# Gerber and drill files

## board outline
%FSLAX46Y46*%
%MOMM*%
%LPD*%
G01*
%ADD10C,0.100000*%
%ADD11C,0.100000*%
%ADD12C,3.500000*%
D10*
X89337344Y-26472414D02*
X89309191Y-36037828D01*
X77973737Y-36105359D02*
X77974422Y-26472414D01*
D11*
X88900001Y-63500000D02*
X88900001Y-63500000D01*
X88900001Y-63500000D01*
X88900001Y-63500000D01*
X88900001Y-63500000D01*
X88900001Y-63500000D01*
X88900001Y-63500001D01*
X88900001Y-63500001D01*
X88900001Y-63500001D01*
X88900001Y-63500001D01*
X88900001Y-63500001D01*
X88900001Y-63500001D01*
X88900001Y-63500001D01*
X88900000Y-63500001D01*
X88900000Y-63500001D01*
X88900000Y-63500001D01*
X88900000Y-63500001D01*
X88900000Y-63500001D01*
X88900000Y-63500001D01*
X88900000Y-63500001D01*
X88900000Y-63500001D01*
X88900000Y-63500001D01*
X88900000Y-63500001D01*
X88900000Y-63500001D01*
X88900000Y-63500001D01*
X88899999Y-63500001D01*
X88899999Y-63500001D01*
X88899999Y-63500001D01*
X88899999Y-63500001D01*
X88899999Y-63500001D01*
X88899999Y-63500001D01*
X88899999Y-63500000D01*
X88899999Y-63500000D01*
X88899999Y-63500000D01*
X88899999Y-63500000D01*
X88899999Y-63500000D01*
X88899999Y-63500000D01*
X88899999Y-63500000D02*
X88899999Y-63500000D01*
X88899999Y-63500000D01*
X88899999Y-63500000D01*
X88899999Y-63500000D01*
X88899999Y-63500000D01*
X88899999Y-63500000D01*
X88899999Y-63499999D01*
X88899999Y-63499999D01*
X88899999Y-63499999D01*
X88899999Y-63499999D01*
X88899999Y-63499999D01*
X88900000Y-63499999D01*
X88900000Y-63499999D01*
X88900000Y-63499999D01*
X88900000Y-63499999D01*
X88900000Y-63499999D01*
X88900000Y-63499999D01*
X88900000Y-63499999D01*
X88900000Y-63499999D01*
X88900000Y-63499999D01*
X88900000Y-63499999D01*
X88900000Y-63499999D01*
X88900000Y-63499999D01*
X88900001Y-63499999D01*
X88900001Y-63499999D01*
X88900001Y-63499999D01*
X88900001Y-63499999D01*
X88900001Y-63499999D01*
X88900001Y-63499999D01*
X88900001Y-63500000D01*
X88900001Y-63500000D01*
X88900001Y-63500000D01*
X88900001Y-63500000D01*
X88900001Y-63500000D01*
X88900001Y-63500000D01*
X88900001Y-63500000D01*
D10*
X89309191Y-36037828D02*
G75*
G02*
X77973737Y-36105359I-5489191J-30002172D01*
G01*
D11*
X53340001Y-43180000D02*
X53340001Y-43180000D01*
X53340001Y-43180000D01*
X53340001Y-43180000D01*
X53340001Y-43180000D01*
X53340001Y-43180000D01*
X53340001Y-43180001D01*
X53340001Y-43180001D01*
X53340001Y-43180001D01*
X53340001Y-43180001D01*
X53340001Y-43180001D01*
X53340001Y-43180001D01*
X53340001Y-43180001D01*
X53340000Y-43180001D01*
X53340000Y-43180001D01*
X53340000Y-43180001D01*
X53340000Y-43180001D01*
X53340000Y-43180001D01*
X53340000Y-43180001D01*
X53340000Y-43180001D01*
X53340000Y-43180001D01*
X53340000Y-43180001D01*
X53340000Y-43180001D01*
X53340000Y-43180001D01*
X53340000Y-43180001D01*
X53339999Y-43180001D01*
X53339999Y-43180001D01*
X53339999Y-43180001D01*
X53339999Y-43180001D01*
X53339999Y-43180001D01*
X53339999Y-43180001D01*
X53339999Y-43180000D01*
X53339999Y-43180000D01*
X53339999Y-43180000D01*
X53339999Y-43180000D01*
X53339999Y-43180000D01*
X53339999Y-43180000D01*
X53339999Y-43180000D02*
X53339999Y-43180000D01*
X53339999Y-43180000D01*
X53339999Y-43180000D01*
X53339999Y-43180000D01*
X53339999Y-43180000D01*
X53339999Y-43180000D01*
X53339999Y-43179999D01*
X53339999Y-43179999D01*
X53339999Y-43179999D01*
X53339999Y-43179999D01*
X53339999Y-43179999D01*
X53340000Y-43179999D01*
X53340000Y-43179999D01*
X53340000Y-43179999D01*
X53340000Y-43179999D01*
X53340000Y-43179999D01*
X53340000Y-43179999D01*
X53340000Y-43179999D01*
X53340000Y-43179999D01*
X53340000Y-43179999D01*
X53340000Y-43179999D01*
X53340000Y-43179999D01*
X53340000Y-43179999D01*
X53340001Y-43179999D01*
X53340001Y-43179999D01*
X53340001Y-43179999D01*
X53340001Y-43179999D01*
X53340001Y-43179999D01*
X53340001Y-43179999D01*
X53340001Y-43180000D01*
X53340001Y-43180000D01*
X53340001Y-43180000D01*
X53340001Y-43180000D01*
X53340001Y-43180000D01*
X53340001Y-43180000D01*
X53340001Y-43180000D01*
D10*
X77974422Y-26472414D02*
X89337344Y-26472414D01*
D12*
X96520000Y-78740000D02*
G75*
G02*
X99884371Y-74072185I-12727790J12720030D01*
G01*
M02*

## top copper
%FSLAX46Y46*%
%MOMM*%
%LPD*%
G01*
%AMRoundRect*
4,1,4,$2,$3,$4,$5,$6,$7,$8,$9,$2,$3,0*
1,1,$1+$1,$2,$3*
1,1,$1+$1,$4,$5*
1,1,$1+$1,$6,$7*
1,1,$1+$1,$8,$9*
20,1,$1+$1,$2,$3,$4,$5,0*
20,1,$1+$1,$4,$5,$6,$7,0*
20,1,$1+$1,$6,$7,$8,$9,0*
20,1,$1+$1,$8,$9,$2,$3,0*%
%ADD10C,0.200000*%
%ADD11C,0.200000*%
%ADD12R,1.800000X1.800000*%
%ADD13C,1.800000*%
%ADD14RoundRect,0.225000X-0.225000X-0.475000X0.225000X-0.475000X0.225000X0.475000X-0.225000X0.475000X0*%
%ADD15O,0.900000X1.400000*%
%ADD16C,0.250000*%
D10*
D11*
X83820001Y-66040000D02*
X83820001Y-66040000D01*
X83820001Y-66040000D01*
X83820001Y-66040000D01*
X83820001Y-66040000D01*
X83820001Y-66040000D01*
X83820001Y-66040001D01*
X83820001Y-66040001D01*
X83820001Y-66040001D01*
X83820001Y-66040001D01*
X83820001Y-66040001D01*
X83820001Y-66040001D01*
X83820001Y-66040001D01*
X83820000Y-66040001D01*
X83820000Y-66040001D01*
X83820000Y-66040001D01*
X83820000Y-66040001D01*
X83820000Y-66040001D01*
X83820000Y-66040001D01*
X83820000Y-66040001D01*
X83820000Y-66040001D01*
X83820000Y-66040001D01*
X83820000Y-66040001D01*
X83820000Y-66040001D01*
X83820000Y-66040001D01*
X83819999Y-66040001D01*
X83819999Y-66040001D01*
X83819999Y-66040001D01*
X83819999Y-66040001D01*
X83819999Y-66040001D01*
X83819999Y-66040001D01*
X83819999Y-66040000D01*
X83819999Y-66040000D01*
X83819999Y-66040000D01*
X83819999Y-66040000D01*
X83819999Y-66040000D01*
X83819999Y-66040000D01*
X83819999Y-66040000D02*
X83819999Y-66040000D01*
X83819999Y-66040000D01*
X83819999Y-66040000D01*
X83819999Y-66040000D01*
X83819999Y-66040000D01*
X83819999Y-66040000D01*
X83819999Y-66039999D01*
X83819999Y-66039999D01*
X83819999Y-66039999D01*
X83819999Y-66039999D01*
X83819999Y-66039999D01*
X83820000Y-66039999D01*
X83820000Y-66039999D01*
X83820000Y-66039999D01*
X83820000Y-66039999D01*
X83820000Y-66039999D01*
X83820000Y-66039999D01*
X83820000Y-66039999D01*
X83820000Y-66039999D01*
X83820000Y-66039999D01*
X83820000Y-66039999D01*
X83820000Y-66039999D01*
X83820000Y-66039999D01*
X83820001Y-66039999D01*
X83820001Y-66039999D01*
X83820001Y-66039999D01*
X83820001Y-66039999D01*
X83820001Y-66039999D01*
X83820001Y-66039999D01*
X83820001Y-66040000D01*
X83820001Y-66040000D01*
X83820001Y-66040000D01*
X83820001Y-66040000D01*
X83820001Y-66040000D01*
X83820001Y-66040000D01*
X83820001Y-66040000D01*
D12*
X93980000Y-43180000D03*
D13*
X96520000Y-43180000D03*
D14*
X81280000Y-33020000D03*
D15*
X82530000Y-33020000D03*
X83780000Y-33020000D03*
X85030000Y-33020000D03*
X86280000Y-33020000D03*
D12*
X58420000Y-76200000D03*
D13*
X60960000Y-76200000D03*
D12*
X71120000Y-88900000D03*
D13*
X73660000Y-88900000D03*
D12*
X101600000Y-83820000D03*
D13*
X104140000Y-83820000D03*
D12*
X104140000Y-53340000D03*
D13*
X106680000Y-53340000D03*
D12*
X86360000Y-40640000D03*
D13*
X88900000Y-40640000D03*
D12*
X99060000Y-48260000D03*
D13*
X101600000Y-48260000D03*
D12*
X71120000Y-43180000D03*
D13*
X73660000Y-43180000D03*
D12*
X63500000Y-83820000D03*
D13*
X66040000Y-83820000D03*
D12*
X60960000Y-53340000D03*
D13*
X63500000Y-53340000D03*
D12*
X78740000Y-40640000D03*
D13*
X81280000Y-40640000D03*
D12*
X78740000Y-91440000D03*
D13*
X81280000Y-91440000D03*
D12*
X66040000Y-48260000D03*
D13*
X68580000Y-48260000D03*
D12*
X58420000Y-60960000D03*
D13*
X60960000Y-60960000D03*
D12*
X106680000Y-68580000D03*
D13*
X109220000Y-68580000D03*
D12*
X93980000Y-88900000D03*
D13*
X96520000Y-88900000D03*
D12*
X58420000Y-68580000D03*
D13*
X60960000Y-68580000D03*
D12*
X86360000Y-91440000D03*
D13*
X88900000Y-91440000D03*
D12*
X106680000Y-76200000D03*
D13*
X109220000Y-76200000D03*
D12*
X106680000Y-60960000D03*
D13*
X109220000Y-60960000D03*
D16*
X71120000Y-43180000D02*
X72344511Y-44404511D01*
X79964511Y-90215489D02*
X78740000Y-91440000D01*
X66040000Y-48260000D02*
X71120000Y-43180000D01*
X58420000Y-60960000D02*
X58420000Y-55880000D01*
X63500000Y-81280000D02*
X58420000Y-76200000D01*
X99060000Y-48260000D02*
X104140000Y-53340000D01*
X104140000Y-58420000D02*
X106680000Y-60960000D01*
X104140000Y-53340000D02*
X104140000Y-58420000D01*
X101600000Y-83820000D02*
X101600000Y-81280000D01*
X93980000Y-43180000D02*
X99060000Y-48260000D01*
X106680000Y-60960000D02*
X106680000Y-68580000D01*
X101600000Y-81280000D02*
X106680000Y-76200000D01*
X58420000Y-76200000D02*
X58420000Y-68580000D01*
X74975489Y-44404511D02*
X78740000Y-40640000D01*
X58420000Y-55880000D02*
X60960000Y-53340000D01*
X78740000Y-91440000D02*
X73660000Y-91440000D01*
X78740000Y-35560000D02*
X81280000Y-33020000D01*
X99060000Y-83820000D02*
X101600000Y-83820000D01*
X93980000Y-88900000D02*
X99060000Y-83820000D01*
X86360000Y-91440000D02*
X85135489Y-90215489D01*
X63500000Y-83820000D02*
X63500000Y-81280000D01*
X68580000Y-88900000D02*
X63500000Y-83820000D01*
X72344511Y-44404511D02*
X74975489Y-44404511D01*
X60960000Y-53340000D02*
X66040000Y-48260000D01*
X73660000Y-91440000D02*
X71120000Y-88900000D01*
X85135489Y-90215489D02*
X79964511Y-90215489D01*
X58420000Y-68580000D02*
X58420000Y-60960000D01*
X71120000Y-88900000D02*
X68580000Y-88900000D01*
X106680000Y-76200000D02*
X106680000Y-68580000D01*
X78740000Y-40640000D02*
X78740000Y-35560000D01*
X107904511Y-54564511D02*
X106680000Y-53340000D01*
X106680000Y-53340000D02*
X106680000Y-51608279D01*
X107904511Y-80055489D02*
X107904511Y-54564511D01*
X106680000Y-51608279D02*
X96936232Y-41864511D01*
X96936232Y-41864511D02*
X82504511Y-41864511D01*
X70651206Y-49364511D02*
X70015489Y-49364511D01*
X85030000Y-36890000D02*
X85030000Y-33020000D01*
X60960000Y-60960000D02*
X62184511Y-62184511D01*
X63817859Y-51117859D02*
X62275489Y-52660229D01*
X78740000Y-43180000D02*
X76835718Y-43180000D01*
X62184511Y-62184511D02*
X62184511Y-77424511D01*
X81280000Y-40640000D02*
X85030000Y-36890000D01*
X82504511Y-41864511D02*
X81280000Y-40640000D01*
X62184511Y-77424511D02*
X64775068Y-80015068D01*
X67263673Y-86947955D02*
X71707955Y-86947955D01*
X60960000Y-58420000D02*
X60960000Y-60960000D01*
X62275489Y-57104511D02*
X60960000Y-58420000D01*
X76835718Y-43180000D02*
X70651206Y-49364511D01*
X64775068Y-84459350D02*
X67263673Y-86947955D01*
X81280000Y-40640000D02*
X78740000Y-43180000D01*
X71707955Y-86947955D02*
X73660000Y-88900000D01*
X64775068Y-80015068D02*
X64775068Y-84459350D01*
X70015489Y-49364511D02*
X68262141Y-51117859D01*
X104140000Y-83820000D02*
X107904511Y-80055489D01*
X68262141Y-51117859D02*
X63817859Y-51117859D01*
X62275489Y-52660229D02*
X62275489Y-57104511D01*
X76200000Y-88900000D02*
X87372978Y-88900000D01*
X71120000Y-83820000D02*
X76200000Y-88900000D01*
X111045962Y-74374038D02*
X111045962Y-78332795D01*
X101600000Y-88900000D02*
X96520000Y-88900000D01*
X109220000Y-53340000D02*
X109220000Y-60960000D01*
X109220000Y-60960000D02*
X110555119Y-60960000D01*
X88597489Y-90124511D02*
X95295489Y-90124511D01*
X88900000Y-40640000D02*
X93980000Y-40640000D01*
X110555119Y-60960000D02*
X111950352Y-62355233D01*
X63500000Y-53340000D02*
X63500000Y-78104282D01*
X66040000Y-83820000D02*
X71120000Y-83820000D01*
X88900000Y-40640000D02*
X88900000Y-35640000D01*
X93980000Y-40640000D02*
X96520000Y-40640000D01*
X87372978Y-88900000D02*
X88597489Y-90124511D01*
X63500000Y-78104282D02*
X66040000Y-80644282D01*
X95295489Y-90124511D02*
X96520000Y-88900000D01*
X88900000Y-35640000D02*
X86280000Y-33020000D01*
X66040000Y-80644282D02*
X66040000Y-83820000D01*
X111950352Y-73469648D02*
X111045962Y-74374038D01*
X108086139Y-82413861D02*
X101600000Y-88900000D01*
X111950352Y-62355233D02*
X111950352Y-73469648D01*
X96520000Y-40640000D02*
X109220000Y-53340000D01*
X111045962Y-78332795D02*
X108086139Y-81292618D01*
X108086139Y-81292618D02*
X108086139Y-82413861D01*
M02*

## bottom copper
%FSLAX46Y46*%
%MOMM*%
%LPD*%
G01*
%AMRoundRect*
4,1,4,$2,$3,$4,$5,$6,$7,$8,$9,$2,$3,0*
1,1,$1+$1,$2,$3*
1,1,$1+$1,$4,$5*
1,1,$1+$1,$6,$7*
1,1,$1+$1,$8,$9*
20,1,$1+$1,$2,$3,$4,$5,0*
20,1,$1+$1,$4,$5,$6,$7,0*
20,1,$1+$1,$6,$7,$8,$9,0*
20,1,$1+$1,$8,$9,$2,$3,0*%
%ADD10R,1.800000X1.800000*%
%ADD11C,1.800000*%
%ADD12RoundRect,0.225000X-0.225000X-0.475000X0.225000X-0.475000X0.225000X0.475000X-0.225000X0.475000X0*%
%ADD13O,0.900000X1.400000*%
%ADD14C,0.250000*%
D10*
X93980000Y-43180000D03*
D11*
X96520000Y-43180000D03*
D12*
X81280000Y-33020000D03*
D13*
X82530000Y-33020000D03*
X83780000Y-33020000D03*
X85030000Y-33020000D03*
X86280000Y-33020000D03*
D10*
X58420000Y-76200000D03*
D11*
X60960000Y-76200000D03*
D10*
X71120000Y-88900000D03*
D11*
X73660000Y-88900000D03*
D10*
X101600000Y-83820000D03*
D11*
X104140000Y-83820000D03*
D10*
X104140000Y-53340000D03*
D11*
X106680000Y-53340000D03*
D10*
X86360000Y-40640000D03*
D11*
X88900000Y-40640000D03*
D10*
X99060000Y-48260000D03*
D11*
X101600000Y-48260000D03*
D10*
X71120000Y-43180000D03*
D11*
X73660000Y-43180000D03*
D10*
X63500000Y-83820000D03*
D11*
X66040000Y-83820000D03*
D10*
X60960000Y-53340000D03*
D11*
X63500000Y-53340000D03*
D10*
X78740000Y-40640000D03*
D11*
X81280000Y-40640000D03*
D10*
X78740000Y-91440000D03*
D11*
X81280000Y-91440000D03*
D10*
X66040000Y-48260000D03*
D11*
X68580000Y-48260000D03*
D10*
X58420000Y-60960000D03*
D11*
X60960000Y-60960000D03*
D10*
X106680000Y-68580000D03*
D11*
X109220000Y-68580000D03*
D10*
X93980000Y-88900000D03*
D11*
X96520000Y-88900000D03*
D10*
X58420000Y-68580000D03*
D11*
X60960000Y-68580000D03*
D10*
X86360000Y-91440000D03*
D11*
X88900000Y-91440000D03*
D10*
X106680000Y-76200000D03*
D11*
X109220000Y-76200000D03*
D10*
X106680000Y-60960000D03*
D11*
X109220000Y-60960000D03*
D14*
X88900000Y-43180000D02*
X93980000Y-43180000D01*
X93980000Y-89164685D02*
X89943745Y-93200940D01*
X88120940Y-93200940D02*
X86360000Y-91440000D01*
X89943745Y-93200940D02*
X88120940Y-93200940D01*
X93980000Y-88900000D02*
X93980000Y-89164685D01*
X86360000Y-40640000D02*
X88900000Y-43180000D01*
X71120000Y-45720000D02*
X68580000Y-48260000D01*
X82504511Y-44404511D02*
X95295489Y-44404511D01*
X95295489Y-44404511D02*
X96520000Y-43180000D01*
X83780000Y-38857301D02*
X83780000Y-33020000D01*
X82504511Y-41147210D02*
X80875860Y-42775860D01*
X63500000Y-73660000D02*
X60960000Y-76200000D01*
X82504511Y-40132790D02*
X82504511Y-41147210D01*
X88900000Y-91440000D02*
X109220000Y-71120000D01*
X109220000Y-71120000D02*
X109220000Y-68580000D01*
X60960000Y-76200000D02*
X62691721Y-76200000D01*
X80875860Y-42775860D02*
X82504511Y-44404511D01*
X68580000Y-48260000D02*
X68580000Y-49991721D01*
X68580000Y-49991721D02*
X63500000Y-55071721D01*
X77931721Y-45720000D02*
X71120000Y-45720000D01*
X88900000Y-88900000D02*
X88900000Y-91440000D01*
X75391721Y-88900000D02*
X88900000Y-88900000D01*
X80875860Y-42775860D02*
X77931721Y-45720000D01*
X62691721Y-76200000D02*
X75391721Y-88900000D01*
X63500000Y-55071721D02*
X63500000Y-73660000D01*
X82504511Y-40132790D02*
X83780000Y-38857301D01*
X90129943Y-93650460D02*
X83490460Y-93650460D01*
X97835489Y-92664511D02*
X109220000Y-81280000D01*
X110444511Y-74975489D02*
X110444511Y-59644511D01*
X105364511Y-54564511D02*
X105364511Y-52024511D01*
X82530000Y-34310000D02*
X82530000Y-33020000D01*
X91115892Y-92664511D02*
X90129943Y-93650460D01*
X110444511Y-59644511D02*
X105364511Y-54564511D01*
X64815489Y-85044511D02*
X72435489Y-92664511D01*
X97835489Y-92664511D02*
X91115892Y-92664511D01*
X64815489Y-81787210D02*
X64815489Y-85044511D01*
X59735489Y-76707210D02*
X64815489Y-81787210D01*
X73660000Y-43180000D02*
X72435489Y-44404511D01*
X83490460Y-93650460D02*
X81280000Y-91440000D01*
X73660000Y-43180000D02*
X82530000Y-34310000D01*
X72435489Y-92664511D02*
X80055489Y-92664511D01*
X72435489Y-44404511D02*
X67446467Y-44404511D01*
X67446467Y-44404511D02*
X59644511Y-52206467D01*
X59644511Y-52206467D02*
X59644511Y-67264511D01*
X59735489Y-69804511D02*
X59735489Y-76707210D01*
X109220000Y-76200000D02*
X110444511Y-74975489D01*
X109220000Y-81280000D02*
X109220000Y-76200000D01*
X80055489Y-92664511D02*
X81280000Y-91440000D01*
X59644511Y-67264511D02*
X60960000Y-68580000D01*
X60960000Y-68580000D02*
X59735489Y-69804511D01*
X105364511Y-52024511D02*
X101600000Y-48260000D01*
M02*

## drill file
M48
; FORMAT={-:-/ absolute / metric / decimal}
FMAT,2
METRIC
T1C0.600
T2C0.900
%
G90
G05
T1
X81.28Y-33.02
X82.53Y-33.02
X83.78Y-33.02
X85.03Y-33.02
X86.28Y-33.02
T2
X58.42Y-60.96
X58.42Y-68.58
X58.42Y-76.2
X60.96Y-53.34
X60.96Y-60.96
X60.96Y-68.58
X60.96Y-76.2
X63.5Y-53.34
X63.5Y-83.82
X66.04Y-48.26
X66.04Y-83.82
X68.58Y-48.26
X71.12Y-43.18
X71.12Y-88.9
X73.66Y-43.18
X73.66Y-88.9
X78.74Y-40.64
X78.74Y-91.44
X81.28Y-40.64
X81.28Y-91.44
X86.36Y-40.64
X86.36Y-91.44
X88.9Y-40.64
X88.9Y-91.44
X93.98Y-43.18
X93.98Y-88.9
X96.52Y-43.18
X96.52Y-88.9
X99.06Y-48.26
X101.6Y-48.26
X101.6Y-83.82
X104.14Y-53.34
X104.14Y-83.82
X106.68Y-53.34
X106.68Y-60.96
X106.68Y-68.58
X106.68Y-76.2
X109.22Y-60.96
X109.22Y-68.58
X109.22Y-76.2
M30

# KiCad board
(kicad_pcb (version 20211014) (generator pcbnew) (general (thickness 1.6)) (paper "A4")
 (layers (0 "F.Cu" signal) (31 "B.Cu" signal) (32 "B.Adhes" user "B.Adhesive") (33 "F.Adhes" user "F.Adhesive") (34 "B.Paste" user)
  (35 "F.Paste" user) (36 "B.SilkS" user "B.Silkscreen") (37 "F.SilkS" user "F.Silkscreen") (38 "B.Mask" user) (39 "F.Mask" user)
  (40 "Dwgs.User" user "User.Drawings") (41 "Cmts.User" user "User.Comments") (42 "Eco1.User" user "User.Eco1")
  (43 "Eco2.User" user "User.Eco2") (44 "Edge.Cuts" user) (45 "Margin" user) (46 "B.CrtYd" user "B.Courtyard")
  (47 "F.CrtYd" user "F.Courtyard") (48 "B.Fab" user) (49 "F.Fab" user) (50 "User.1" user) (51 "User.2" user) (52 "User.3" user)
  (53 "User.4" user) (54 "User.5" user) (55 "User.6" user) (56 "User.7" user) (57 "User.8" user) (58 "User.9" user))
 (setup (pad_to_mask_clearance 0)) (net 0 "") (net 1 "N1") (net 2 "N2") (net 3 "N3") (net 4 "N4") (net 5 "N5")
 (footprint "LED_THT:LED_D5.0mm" (layer "F.Cu") (at 93.98 43.18)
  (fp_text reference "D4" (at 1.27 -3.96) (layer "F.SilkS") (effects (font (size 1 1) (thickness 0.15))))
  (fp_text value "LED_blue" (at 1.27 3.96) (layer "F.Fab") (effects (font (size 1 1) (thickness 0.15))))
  (pad "1" thru_hole rect (at 0 0) (size 1.8 1.8) (drill 0.9) (layers *.Cu *.Mask) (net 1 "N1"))
  (pad "2" thru_hole circle (at 2.54 0) (size 1.8 1.8) (drill 0.9) (layers *.Cu *.Mask) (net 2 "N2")))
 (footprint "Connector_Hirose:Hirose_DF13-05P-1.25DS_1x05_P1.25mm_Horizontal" (layer "F.Cu") (at 81.28 33.02)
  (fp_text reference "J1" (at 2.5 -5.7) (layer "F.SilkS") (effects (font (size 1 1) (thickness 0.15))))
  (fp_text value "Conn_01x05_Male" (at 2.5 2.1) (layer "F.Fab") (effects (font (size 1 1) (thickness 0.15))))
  (pad "1" thru_hole roundrect (at 0 0) (size 0.9 1.4) (drill 0.6) (layers *.Cu *.Mask) (roundrect_rratio 0.25) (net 1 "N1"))
  (pad "2" thru_hole oval (at 1.25 0) (size 0.9 1.4) (drill 0.6) (layers *.Cu *.Mask) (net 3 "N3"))
  (pad "3" thru_hole oval (at 2.5 0) (size 0.9 1.4) (drill 0.6) (layers *.Cu *.Mask) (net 2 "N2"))
  (pad "4" thru_hole oval (at 3.75 0) (size 0.9 1.4) (drill 0.6) (layers *.Cu *.Mask) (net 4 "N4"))
  (pad "5" thru_hole oval (at 5 0) (size 0.9 1.4) (drill 0.6) (layers *.Cu *.Mask) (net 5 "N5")))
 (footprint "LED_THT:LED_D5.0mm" (layer "F.Cu") (at 58.42 76.2)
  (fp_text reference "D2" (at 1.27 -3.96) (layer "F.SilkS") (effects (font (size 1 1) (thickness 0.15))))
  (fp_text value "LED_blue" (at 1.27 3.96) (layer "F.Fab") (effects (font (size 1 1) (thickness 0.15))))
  (pad "1" thru_hole rect (at 0 0) (size 1.8 1.8) (drill 0.9) (layers *.Cu *.Mask) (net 1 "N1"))
  (pad "2" thru_hole circle (at 2.54 0) (size 1.8 1.8) (drill 0.9) (layers *.Cu *.Mask) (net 2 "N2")))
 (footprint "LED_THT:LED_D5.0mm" (layer "F.Cu") (at 71.12 88.9)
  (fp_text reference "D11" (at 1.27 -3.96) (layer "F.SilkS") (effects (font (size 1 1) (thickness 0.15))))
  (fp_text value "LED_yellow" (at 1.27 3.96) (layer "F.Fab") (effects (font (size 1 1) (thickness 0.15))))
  (pad "1" thru_hole rect (at 0 0) (size 1.8 1.8) (drill 0.9) (layers *.Cu *.Mask) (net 1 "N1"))
  (pad "2" thru_hole circle (at 2.54 0) (size 1.8 1.8) (drill 0.9) (layers *.Cu *.Mask) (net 4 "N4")))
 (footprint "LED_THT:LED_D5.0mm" (layer "F.Cu") (at 101.6 83.82)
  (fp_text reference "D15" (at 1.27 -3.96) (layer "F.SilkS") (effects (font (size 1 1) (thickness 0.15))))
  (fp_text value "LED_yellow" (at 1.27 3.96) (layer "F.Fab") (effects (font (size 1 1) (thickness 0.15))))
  (pad "1" thru_hole rect (at 0 0) (size 1.8 1.8) (drill 0.9) (layers *.Cu *.Mask) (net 1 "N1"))
  (pad "2" thru_hole circle (at 2.54 0) (size 1.8 1.8) (drill 0.9) (layers *.Cu *.Mask) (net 4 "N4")))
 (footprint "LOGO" (layer "F.Cu") (at 54.881544 65.757598 90)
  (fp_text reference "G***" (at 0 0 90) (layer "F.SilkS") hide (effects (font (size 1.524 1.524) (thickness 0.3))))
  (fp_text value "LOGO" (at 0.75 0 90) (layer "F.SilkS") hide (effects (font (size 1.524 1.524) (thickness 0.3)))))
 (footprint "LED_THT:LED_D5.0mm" (layer "F.Cu") (at 104.14 53.34)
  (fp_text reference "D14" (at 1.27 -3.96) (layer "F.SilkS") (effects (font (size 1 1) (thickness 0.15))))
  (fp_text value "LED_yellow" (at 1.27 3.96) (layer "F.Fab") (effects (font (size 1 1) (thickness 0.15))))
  (pad "1" thru_hole rect (at 0 0) (size 1.8 1.8) (drill 0.9) (layers *.Cu *.Mask) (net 1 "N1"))
  (pad "2" thru_hole circle (at 2.54 0) (size 1.8 1.8) (drill 0.9) (layers *.Cu *.Mask) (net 4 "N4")))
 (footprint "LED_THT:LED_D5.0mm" (layer "F.Cu") (at 86.36 40.64)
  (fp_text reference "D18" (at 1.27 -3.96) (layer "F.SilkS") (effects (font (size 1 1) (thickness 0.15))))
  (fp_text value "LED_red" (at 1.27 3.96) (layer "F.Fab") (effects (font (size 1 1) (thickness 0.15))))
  (pad "1" thru_hole rect (at 0 0) (size 1.8 1.8) (drill 0.9) (layers *.Cu *.Mask) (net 1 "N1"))
  (pad "2" thru_hole circle (at 2.54 0) (size 1.8 1.8) (drill 0.9) (layers *.Cu *.Mask) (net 5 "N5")))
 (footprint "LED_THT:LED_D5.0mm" (layer "F.Cu") (at 99.06 48.26)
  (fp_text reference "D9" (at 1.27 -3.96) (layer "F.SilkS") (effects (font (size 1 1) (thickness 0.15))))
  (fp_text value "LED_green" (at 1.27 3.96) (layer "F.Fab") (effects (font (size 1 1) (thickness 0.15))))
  (pad "1" thru_hole rect (at 0 0) (size 1.8 1.8) (drill 0.9) (layers *.Cu *.Mask) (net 1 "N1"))
  (pad "2" thru_hole circle (at 2.54 0) (size 1.8 1.8) (drill 0.9) (layers *.Cu *.Mask) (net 3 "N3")))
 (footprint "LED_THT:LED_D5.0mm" (layer "F.Cu") (at 71.12 43.18)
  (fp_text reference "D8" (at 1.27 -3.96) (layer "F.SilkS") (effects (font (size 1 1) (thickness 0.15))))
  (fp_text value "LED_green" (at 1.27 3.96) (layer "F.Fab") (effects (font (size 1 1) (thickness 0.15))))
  (pad "1" thru_hole rect (at 0 0) (size 1.8 1.8) (drill 0.9) (layers *.Cu *.Mask) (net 1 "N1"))
  (pad "2" thru_hole circle (at 2.54 0) (size 1.8 1.8) (drill 0.9) (layers *.Cu *.Mask) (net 3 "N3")))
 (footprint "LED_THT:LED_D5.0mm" (layer "F.Cu") (at 63.5 83.82)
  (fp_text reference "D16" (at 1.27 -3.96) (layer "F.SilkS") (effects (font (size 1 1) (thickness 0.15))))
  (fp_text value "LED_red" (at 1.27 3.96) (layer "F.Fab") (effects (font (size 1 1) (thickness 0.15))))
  (pad "1" thru_hole rect (at 0 0) (size 1.8 1.8) (drill 0.9) (layers *.Cu *.Mask) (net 1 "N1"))
  (pad "2" thru_hole circle (at 2.54 0) (size 1.8 1.8) (drill 0.9) (layers *.Cu *.Mask) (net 5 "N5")))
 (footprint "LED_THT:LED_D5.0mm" (layer "F.Cu") (at 60.96 53.34)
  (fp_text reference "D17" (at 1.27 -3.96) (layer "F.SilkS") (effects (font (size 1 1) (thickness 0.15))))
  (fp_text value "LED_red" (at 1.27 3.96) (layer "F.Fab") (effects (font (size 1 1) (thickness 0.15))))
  (pad "1" thru_hole rect (at 0 0) (size 1.8 1.8) (drill 0.9) (layers *.Cu *.Mask) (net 1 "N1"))
  (pad "2" thru_hole circle (at 2.54 0) (size 1.8 1.8) (drill 0.9) (layers *.Cu *.Mask) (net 5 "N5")))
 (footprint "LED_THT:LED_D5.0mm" (layer "F.Cu") (at 78.74 40.64)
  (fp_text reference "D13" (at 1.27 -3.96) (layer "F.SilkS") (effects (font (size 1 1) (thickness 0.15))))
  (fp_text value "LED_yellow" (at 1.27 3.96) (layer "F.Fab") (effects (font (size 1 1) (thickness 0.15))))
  (pad "1" thru_hole rect (at 0 0) (size 1.8 1.8) (drill 0.9) (layers *.Cu *.Mask) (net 1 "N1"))
  (pad "2" thru_hole circle (at 2.54 0) (size 1.8 1.8) (drill 0.9) (layers *.Cu *.Mask) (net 4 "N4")))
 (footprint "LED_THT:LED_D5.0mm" (layer "F.Cu") (at 78.74 91.44)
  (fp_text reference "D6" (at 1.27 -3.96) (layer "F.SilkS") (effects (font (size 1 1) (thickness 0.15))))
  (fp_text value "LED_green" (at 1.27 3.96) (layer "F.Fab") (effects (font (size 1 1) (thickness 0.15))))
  (pad "1" thru_hole rect (at 0 0) (size 1.8 1.8) (drill 0.9) (layers *.Cu *.Mask) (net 1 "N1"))
  (pad "2" thru_hole circle (at 2.54 0) (size 1.8 1.8) (drill 0.9) (layers *.Cu *.Mask) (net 3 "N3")))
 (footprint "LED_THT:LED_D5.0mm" (layer "F.Cu") (at 66.04 48.26)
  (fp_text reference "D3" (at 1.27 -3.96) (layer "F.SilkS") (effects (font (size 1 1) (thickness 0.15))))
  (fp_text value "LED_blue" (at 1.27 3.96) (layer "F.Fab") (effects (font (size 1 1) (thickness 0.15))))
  (pad "1" thru_hole rect (at 0 0) (size 1.8 1.8) (drill 0.9) (layers *.Cu *.Mask) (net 1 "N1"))
  (pad "2" thru_hole circle (at 2.54 0) (size 1.8 1.8) (drill 0.9) (layers *.Cu *.Mask) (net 2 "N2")))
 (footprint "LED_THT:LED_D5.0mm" (layer "F.Cu") (at 58.42 60.96)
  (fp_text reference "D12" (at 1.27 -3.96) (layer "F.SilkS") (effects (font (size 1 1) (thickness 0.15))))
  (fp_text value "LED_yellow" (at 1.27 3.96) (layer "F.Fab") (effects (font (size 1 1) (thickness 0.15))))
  (pad "1" thru_hole rect (at 0 0) (size 1.8 1.8) (drill 0.9) (layers *.Cu *.Mask) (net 1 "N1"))
  (pad "2" thru_hole circle (at 2.54 0) (size 1.8 1.8) (drill 0.9) (layers *.Cu *.Mask) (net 4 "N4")))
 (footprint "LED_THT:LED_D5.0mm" (layer "F.Cu") (at 106.68 68.58)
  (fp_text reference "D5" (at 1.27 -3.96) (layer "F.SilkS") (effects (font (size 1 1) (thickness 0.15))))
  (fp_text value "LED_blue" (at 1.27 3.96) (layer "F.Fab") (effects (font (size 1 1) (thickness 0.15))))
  (pad "1" thru_hole rect (at 0 0) (size 1.8 1.8) (drill 0.9) (layers *.Cu *.Mask) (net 1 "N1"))
  (pad "2" thru_hole circle (at 2.54 0) (size 1.8 1.8) (drill 0.9) (layers *.Cu *.Mask) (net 2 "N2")))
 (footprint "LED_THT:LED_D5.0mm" (layer "F.Cu") (at 93.98 88.9)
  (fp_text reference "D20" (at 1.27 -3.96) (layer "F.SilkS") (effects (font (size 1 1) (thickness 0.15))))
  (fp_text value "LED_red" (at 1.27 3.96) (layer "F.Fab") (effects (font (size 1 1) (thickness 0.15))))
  (pad "1" thru_hole rect (at 0 0) (size 1.8 1.8) (drill 0.9) (layers *.Cu *.Mask) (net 1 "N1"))
  (pad "2" thru_hole circle (at 2.54 0) (size 1.8 1.8) (drill 0.9) (layers *.Cu *.Mask) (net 5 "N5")))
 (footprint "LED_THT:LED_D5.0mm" (layer "F.Cu") (at 58.42 68.58)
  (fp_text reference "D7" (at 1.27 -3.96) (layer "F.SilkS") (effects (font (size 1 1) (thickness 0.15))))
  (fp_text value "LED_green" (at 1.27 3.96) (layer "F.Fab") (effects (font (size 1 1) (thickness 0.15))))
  (pad "1" thru_hole rect (at 0 0) (size 1.8 1.8) (drill 0.9) (layers *.Cu *.Mask) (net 1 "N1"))
  (pad "2" thru_hole circle (at 2.54 0) (size 1.8 1.8) (drill 0.9) (layers *.Cu *.Mask) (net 3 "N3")))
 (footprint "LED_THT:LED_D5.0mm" (layer "F.Cu") (at 86.36 91.44)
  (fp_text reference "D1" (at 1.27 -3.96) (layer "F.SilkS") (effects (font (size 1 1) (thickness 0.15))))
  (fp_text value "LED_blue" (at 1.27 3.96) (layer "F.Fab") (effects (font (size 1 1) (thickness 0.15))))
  (pad "1" thru_hole rect (at 0 0) (size 1.8 1.8) (drill 0.9) (layers *.Cu *.Mask) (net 1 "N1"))
  (pad "2" thru_hole circle (at 2.54 0) (size 1.8 1.8) (drill 0.9) (layers *.Cu *.Mask) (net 2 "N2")))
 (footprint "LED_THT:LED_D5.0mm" (layer "F.Cu") (at 106.68 76.2)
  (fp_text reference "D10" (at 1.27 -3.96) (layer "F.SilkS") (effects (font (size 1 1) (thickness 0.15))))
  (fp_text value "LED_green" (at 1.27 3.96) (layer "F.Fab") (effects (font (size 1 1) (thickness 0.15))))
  (pad "1" thru_hole rect (at 0 0) (size 1.8 1.8) (drill 0.9) (layers *.Cu *.Mask) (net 1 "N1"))
  (pad "2" thru_hole circle (at 2.54 0) (size 1.8 1.8) (drill 0.9) (layers *.Cu *.Mask) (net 3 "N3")))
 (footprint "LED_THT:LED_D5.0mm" (layer "F.Cu") (at 106.68 60.96)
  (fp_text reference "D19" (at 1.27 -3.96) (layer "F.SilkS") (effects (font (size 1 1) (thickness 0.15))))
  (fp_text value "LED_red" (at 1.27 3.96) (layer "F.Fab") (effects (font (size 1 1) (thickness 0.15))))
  (pad "1" thru_hole rect (at 0 0) (size 1.8 1.8) (drill 0.9) (layers *.Cu *.Mask) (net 1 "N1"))
  (pad "2" thru_hole circle (at 2.54 0) (size 1.8 1.8) (drill 0.9) (layers *.Cu *.Mask) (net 5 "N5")))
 (gr_circle (center 83.82 66.04) (end 83.82 66.04) (layer "F.Cu") (width 0.2) (fill none))
 (gr_line (start 89.337344 26.472414) (end 89.309191 36.037828) (layer "Edge.Cuts") (width 0.1))
 (gr_line (start 77.973737 36.105359) (end 77.974422 26.472414) (layer "Edge.Cuts") (width 0.1))
 (gr_circle (center 88.9 63.5) (end 88.9 63.5) (layer "Edge.Cuts") (width 0.1) (fill none))
 (gr_arc (start 89.309191 36.037828) (mid 84.001703 96.539648) (end 77.973737 36.105359) (layer "Edge.Cuts") (width 0.1))
 (gr_circle (center 53.34 43.18) (end 53.34 43.18) (layer "Edge.Cuts") (width 0.1) (fill none))
 (gr_line (start 77.974422 26.472414) (end 89.337344 26.472414) (layer "Edge.Cuts") (width 0.1))
 (gr_arc (start 96.52 78.74) (mid 69.194443 55.4985) (end 99.88437 74.072185) (layer "Edge.Cuts") (width 3.5))
 (segment (start 71.12 43.18) (end 72.344511 44.404511) (width 0.25) (layer "F.Cu") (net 1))
 (segment (start 79.964511 90.215489) (end 78.74 91.44) (width 0.25) (layer "F.Cu") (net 1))
 (segment (start 66.04 48.26) (end 71.12 43.18) (width 0.25) (layer "F.Cu") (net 1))
 (segment (start 58.42 60.96) (end 58.42 55.88) (width 0.25) (layer "F.Cu") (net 1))
 (segment (start 63.5 81.28) (end 58.42 76.2) (width 0.25) (layer "F.Cu") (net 1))
 (segment (start 99.06 48.26) (end 104.14 53.34) (width 0.25) (layer "F.Cu") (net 1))
 (segment (start 104.14 58.42) (end 106.68 60.96) (width 0.25) (layer "F.Cu") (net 1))
 (segment (start 104.14 53.34) (end 104.14 58.42) (width 0.25) (layer "F.Cu") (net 1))
 (segment (start 101.6 83.82) (end 101.6 81.28) (width 0.25) (layer "F.Cu") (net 1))
 (segment (start 93.98 43.18) (end 99.06 48.26) (width 0.25) (layer "F.Cu") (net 1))
 (segment (start 106.68 60.96) (end 106.68 68.58) (width 0.25) (layer "F.Cu") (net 1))
 (segment (start 101.6 81.28) (end 106.68 76.2) (width 0.25) (layer "F.Cu") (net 1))
 (segment (start 58.42 76.2) (end 58.42 68.58) (width 0.25) (layer "F.Cu") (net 1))
 (segment (start 74.975489 44.404511) (end 78.74 40.64) (width 0.25) (layer "F.Cu") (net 1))
 (segment (start 58.42 55.88) (end 60.96 53.34) (width 0.25) (layer "F.Cu") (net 1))
 (segment (start 78.74 91.44) (end 73.66 91.44) (width 0.25) (layer "F.Cu") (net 1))
 (segment (start 78.74 35.56) (end 81.28 33.02) (width 0.25) (layer "F.Cu") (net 1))
 (segment (start 99.06 83.82) (end 101.6 83.82) (width 0.25) (layer "F.Cu") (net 1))
 (segment (start 93.98 88.9) (end 99.06 83.82) (width 0.25) (layer "F.Cu") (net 1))
 (segment (start 86.36 91.44) (end 85.135489 90.215489) (width 0.25) (layer "F.Cu") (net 1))
 (segment (start 63.5 83.82) (end 63.5 81.28) (width 0.25) (layer "F.Cu") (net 1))
 (segment (start 68.58 88.9) (end 63.5 83.82) (width 0.25) (layer "F.Cu") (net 1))
 (segment (start 72.344511 44.404511) (end 74.975489 44.404511) (width 0.25) (layer "F.Cu") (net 1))
 (segment (start 60.96 53.34) (end 66.04 48.26) (width 0.25) (layer "F.Cu") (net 1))
 (segment (start 73.66 91.44) (end 71.12 88.9) (width 0.25) (layer "F.Cu") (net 1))
 (segment (start 85.135489 90.215489) (end 79.964511 90.215489) (width 0.25) (layer "F.Cu") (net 1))
 (segment (start 58.42 68.58) (end 58.42 60.96) (width 0.25) (layer "F.Cu") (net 1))
 (segment (start 71.12 88.9) (end 68.58 88.9) (width 0.25) (layer "F.Cu") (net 1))
 (segment (start 106.68 76.2) (end 106.68 68.58) (width 0.25) (layer "F.Cu") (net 1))
 (segment (start 78.74 40.64) (end 78.74 35.56) (width 0.25) (layer "F.Cu") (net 1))
 (segment (start 88.9 43.18) (end 93.98 43.18) (width 0.25) (layer "B.Cu") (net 1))
 (segment (start 93.98 89.164685) (end 89.943745 93.20094) (width 0.25) (layer "B.Cu") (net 1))
 (segment (start 88.12094 93.20094) (end 86.36 91.44) (width 0.25) (layer "B.Cu") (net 1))
 (segment (start 89.943745 93.20094) (end 88.12094 93.20094) (width 0.25) (layer "B.Cu") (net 1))
 (segment (start 93.98 88.9) (end 93.98 89.164685) (width 0.25) (layer "B.Cu") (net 1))
 (segment (start 86.36 40.64) (end 88.9 43.18) (width 0.25) (layer "B.Cu") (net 1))
 (segment (start 71.12 45.72) (end 68.58 48.26) (width 0.25) (layer "B.Cu") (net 2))
 (segment (start 82.504511 44.404511) (end 95.295489 44.404511) (width 0.25) (layer "B.Cu") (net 2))
 (segment (start 95.295489 44.404511) (end 96.52 43.18) (width 0.25) (layer "B.Cu") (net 2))
 (segment (start 83.78 38.857301) (end 83.78 33.02) (width 0.25) (layer "B.Cu") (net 2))
 (segment (start 82.504511 41.14721) (end 80.87586 42.77586) (width 0.25) (layer "B.Cu") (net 2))
 (segment (start 63.5 73.66) (end 60.96 76.2) (width 0.25) (layer "B.Cu") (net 2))
 (segment (start 82.504511 40.13279) (end 82.504511 41.14721) (width 0.25) (layer "B.Cu") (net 2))
 (segment (start 88.9 91.44) (end 109.22 71.12) (width 0.25) (layer "B.Cu") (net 2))
 (segment (start 109.22 71.12) (end 109.22 68.58) (width 0.25) (layer "B.Cu") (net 2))
 (segment (start 60.96 76.2) (end 62.691721 76.2) (width 0.25) (layer "B.Cu") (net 2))
 (segment (start 80.87586 42.77586) (end 82.504511 44.404511) (width 0.25) (layer "B.Cu") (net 2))
 (segment (start 68.58 48.26) (end 68.58 49.991721) (width 0.25) (layer "B.Cu") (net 2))
 (segment (start 68.58 49.991721) (end 63.5 55.071721) (width 0.25) (layer "B.Cu") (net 2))
 (segment (start 77.931721 45.72) (end 71.12 45.72) (width 0.25) (layer "B.Cu") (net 2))
 (segment (start 88.9 88.9) (end 88.9 91.44) (width 0.25) (layer "B.Cu") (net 2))
 (segment (start 75.391721 88.9) (end 88.9 88.9) (width 0.25) (layer "B.Cu") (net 2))
 (segment (start 80.87586 42.77586) (end 77.931721 45.72) (width 0.25) (layer "B.Cu") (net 2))
 (segment (start 62.691721 76.2) (end 75.391721 88.9) (width 0.25) (layer "B.Cu") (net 2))
 (segment (start 63.5 55.071721) (end 63.5 73.66) (width 0.25) (layer "B.Cu") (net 2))
 (segment (start 82.504511 40.13279) (end 83.78 38.857301) (width 0.25) (layer "B.Cu") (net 2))
 (segment (start 90.129943 93.65046) (end 83.49046 93.65046) (width 0.25) (layer "B.Cu") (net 3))
 (segment (start 97.835489 92.664511) (end 109.22 81.28) (width 0.25) (layer "B.Cu") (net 3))
 (segment (start 110.444511 74.975489) (end 110.444511 59.644511) (width 0.25) (layer "B.Cu") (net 3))
 (segment (start 105.364511 54.564511) (end 105.364511 52.024511) (width 0.25) (layer "B.Cu") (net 3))
 (segment (start 82.53 34.31) (end 82.53 33.02) (width 0.25) (layer "B.Cu") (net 3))
 (segment (start 91.115892 92.664511) (end 90.129943 93.65046) (width 0.25) (layer "B.Cu") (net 3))
 (segment (start 110.444511 59.644511) (end 105.364511 54.564511) (width 0.25) (layer "B.Cu") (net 3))
 (segment (start 64.815489 85.044511) (end 72.435489 92.664511) (width 0.25) (layer "B.Cu") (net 3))
 (segment (start 97.835489 92.664511) (end 91.115892 92.664511) (width 0.25) (layer "B.Cu") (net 3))
 (segment (start 64.815489 81.78721) (end 64.815489 85.044511) (width 0.25) (layer "B.Cu") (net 3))
 (segment (start 59.735489 76.70721) (end 64.815489 81.78721) (width 0.25) (layer "B.Cu") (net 3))
 (segment (start 73.66 43.18) (end 72.435489 44.404511) (width 0.25) (layer "B.Cu") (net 3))
 (segment (start 83.49046 93.65046) (end 81.28 91.44) (width 0.25) (layer "B.Cu") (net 3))
 (segment (start 73.66 43.18) (end 82.53 34.31) (width 0.25) (layer "B.Cu") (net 3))
 (segment (start 72.435489 92.664511) (end 80.055489 92.664511) (width 0.25) (layer "B.Cu") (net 3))
 (segment (start 72.435489 44.404511) (end 67.446467 44.404511) (width 0.25) (layer "B.Cu") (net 3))
 (segment (start 67.446467 44.404511) (end 59.644511 52.206467) (width 0.25) (layer "B.Cu") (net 3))
 (segment (start 59.644511 52.206467) (end 59.644511 67.264511) (width 0.25) (layer "B.Cu") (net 3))
 (segment (start 59.735489 69.804511) (end 59.735489 76.70721) (width 0.25) (layer "B.Cu") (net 3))
 (segment (start 109.22 76.2) (end 110.444511 74.975489) (width 0.25) (layer "B.Cu") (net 3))
 (segment (start 109.22 81.28) (end 109.22 76.2) (width 0.25) (layer "B.Cu") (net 3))
 (segment (start 80.055489 92.664511) (end 81.28 91.44) (width 0.25) (layer "B.Cu") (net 3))
 (segment (start 59.644511 67.264511) (end 60.96 68.58) (width 0.25) (layer "B.Cu") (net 3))
 (segment (start 60.96 68.58) (end 59.735489 69.804511) (width 0.25) (layer "B.Cu") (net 3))
 (segment (start 105.364511 52.024511) (end 101.6 48.26) (width 0.25) (layer "B.Cu") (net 3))
 (segment (start 107.904511 54.564511) (end 106.68 53.34) (width 0.25) (layer "F.Cu") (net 4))
 (segment (start 106.68 53.34) (end 106.68 51.608279) (width 0.25) (layer "F.Cu") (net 4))
 (segment (start 107.904511 80.055489) (end 107.904511 54.564511) (width 0.25) (layer "F.Cu") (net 4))
 (segment (start 106.68 51.608279) (end 96.936232 41.864511) (width 0.25) (layer "F.Cu") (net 4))
 (segment (start 96.936232 41.864511) (end 82.504511 41.864511) (width 0.25) (layer "F.Cu") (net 4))
 (segment (start 70.651206 49.364511) (end 70.015489 49.364511) (width 0.25) (layer "F.Cu") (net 4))
 (segment (start 85.03 36.89) (end 85.03 33.02) (width 0.25) (layer "F.Cu") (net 4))
 (segment (start 60.96 60.96) (end 62.184511 62.184511) (width 0.25) (layer "F.Cu") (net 4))
 (segment (start 63.817859 51.117859) (end 62.275489 52.660229) (width 0.25) (layer "F.Cu") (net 4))
 (segment (start 78.74 43.18) (end 76.835718 43.18) (width 0.25) (layer "F.Cu") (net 4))
 (segment (start 62.184511 62.184511) (end 62.184511 77.424511) (width 0.25) (layer "F.Cu") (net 4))
 (segment (start 81.28 40.64) (end 85.03 36.89) (width 0.25) (layer "F.Cu") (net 4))
 (segment (start 82.504511 41.864511) (end 81.28 40.64) (width 0.25) (layer "F.Cu") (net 4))
 (segment (start 62.184511 77.424511) (end 64.775068 80.015068) (width 0.25) (layer "F.Cu") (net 4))
 (segment (start 67.263673 86.947955) (end 71.707955 86.947955) (width 0.25) (layer "F.Cu") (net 4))
 (segment (start 60.96 58.42) (end 60.96 60.96) (width 0.25) (layer "F.Cu") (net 4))
 (segment (start 62.275489 57.104511) (end 60.96 58.42) (width 0.25) (layer "F.Cu") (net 4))
 (segment (start 76.835718 43.18) (end 70.651206 49.364511) (width 0.25) (layer "F.Cu") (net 4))
 (segment (start 64.775068 84.45935) (end 67.263673 86.947955) (width 0.25) (layer "F.Cu") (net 4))
 (segment (start 81.28 40.64) (end 78.74 43.18) (width 0.25) (layer "F.Cu") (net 4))
 (segment (start 71.707955 86.947955) (end 73.66 88.9) (width 0.25) (layer "F.Cu") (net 4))
 (segment (start 64.775068 80.015068) (end 64.775068 84.45935) (width 0.25) (layer "F.Cu") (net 4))
 (segment (start 70.015489 49.364511) (end 68.262141 51.117859) (width 0.25) (layer "F.Cu") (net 4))
 (segment (start 104.14 83.82) (end 107.904511 80.055489) (width 0.25) (layer "F.Cu") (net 4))
 (segment (start 68.262141 51.117859) (end 63.817859 51.117859) (width 0.25) (layer "F.Cu") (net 4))
 (segment (start 62.275489 52.660229) (end 62.275489 57.104511) (width 0.25) (layer "F.Cu") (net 4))
 (segment (start 76.2 88.9) (end 87.372978 88.9) (width 0.25) (layer "F.Cu") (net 5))
 (segment (start 71.12 83.82) (end 76.2 88.9) (width 0.25) (layer "F.Cu") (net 5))
 (segment (start 111.045962 74.374038) (end 111.045962 78.332795) (width 0.25) (layer "F.Cu") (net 5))
 (segment (start 101.6 88.9) (end 96.52 88.9) (width 0.25) (layer "F.Cu") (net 5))
 (segment (start 109.22 53.34) (end 109.22 60.96) (width 0.25) (layer "F.Cu") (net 5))
 (segment (start 109.22 60.96) (end 110.555119 60.96) (width 0.25) (layer "F.Cu") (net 5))
 (segment (start 88.597489 90.124511) (end 95.295489 90.124511) (width 0.25) (layer "F.Cu") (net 5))
 (segment (start 88.9 40.64) (end 93.98 40.64) (width 0.25) (layer "F.Cu") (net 5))
 (segment (start 110.555119 60.96) (end 111.950352 62.355233) (width 0.25) (layer "F.Cu") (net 5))
 (segment (start 63.5 53.34) (end 63.5 78.104282) (width 0.25) (layer "F.Cu") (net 5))
 (segment (start 66.04 83.82) (end 71.12 83.82) (width 0.25) (layer "F.Cu") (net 5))
 (segment (start 88.9 40.64) (end 88.9 35.64) (width 0.25) (layer "F.Cu") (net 5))
 (segment (start 93.98 40.64) (end 96.52 40.64) (width 0.25) (layer "F.Cu") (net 5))
 (segment (start 87.372978 88.9) (end 88.597489 90.124511) (width 0.25) (layer "F.Cu") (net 5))
 (segment (start 63.5 78.104282) (end 66.04 80.644282) (width 0.25) (layer "F.Cu") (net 5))
 (segment (start 95.295489 90.124511) (end 96.52 88.9) (width 0.25) (layer "F.Cu") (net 5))
 (segment (start 88.9 35.64) (end 86.28 33.02) (width 0.25) (layer "F.Cu") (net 5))
 (segment (start 66.04 80.644282) (end 66.04 83.82) (width 0.25) (layer "F.Cu") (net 5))
 (segment (start 111.950352 73.469648) (end 111.045962 74.374038) (width 0.25) (layer "F.Cu") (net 5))
 (segment (start 108.086139 82.413861) (end 101.6 88.9) (width 0.25) (layer "F.Cu") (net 5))
 (segment (start 111.950352 62.355233) (end 111.950352 73.469648) (width 0.25) (layer "F.Cu") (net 5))
 (segment (start 96.52 40.64) (end 109.22 53.34) (width 0.25) (layer "F.Cu") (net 5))
 (segment (start 111.045962 78.332795) (end 108.086139 81.292618) (width 0.25) (layer "F.Cu") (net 5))
 (segment (start 108.086139 81.292618) (end 108.086139 82.413861) (width 0.25) (layer "F.Cu") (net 5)))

